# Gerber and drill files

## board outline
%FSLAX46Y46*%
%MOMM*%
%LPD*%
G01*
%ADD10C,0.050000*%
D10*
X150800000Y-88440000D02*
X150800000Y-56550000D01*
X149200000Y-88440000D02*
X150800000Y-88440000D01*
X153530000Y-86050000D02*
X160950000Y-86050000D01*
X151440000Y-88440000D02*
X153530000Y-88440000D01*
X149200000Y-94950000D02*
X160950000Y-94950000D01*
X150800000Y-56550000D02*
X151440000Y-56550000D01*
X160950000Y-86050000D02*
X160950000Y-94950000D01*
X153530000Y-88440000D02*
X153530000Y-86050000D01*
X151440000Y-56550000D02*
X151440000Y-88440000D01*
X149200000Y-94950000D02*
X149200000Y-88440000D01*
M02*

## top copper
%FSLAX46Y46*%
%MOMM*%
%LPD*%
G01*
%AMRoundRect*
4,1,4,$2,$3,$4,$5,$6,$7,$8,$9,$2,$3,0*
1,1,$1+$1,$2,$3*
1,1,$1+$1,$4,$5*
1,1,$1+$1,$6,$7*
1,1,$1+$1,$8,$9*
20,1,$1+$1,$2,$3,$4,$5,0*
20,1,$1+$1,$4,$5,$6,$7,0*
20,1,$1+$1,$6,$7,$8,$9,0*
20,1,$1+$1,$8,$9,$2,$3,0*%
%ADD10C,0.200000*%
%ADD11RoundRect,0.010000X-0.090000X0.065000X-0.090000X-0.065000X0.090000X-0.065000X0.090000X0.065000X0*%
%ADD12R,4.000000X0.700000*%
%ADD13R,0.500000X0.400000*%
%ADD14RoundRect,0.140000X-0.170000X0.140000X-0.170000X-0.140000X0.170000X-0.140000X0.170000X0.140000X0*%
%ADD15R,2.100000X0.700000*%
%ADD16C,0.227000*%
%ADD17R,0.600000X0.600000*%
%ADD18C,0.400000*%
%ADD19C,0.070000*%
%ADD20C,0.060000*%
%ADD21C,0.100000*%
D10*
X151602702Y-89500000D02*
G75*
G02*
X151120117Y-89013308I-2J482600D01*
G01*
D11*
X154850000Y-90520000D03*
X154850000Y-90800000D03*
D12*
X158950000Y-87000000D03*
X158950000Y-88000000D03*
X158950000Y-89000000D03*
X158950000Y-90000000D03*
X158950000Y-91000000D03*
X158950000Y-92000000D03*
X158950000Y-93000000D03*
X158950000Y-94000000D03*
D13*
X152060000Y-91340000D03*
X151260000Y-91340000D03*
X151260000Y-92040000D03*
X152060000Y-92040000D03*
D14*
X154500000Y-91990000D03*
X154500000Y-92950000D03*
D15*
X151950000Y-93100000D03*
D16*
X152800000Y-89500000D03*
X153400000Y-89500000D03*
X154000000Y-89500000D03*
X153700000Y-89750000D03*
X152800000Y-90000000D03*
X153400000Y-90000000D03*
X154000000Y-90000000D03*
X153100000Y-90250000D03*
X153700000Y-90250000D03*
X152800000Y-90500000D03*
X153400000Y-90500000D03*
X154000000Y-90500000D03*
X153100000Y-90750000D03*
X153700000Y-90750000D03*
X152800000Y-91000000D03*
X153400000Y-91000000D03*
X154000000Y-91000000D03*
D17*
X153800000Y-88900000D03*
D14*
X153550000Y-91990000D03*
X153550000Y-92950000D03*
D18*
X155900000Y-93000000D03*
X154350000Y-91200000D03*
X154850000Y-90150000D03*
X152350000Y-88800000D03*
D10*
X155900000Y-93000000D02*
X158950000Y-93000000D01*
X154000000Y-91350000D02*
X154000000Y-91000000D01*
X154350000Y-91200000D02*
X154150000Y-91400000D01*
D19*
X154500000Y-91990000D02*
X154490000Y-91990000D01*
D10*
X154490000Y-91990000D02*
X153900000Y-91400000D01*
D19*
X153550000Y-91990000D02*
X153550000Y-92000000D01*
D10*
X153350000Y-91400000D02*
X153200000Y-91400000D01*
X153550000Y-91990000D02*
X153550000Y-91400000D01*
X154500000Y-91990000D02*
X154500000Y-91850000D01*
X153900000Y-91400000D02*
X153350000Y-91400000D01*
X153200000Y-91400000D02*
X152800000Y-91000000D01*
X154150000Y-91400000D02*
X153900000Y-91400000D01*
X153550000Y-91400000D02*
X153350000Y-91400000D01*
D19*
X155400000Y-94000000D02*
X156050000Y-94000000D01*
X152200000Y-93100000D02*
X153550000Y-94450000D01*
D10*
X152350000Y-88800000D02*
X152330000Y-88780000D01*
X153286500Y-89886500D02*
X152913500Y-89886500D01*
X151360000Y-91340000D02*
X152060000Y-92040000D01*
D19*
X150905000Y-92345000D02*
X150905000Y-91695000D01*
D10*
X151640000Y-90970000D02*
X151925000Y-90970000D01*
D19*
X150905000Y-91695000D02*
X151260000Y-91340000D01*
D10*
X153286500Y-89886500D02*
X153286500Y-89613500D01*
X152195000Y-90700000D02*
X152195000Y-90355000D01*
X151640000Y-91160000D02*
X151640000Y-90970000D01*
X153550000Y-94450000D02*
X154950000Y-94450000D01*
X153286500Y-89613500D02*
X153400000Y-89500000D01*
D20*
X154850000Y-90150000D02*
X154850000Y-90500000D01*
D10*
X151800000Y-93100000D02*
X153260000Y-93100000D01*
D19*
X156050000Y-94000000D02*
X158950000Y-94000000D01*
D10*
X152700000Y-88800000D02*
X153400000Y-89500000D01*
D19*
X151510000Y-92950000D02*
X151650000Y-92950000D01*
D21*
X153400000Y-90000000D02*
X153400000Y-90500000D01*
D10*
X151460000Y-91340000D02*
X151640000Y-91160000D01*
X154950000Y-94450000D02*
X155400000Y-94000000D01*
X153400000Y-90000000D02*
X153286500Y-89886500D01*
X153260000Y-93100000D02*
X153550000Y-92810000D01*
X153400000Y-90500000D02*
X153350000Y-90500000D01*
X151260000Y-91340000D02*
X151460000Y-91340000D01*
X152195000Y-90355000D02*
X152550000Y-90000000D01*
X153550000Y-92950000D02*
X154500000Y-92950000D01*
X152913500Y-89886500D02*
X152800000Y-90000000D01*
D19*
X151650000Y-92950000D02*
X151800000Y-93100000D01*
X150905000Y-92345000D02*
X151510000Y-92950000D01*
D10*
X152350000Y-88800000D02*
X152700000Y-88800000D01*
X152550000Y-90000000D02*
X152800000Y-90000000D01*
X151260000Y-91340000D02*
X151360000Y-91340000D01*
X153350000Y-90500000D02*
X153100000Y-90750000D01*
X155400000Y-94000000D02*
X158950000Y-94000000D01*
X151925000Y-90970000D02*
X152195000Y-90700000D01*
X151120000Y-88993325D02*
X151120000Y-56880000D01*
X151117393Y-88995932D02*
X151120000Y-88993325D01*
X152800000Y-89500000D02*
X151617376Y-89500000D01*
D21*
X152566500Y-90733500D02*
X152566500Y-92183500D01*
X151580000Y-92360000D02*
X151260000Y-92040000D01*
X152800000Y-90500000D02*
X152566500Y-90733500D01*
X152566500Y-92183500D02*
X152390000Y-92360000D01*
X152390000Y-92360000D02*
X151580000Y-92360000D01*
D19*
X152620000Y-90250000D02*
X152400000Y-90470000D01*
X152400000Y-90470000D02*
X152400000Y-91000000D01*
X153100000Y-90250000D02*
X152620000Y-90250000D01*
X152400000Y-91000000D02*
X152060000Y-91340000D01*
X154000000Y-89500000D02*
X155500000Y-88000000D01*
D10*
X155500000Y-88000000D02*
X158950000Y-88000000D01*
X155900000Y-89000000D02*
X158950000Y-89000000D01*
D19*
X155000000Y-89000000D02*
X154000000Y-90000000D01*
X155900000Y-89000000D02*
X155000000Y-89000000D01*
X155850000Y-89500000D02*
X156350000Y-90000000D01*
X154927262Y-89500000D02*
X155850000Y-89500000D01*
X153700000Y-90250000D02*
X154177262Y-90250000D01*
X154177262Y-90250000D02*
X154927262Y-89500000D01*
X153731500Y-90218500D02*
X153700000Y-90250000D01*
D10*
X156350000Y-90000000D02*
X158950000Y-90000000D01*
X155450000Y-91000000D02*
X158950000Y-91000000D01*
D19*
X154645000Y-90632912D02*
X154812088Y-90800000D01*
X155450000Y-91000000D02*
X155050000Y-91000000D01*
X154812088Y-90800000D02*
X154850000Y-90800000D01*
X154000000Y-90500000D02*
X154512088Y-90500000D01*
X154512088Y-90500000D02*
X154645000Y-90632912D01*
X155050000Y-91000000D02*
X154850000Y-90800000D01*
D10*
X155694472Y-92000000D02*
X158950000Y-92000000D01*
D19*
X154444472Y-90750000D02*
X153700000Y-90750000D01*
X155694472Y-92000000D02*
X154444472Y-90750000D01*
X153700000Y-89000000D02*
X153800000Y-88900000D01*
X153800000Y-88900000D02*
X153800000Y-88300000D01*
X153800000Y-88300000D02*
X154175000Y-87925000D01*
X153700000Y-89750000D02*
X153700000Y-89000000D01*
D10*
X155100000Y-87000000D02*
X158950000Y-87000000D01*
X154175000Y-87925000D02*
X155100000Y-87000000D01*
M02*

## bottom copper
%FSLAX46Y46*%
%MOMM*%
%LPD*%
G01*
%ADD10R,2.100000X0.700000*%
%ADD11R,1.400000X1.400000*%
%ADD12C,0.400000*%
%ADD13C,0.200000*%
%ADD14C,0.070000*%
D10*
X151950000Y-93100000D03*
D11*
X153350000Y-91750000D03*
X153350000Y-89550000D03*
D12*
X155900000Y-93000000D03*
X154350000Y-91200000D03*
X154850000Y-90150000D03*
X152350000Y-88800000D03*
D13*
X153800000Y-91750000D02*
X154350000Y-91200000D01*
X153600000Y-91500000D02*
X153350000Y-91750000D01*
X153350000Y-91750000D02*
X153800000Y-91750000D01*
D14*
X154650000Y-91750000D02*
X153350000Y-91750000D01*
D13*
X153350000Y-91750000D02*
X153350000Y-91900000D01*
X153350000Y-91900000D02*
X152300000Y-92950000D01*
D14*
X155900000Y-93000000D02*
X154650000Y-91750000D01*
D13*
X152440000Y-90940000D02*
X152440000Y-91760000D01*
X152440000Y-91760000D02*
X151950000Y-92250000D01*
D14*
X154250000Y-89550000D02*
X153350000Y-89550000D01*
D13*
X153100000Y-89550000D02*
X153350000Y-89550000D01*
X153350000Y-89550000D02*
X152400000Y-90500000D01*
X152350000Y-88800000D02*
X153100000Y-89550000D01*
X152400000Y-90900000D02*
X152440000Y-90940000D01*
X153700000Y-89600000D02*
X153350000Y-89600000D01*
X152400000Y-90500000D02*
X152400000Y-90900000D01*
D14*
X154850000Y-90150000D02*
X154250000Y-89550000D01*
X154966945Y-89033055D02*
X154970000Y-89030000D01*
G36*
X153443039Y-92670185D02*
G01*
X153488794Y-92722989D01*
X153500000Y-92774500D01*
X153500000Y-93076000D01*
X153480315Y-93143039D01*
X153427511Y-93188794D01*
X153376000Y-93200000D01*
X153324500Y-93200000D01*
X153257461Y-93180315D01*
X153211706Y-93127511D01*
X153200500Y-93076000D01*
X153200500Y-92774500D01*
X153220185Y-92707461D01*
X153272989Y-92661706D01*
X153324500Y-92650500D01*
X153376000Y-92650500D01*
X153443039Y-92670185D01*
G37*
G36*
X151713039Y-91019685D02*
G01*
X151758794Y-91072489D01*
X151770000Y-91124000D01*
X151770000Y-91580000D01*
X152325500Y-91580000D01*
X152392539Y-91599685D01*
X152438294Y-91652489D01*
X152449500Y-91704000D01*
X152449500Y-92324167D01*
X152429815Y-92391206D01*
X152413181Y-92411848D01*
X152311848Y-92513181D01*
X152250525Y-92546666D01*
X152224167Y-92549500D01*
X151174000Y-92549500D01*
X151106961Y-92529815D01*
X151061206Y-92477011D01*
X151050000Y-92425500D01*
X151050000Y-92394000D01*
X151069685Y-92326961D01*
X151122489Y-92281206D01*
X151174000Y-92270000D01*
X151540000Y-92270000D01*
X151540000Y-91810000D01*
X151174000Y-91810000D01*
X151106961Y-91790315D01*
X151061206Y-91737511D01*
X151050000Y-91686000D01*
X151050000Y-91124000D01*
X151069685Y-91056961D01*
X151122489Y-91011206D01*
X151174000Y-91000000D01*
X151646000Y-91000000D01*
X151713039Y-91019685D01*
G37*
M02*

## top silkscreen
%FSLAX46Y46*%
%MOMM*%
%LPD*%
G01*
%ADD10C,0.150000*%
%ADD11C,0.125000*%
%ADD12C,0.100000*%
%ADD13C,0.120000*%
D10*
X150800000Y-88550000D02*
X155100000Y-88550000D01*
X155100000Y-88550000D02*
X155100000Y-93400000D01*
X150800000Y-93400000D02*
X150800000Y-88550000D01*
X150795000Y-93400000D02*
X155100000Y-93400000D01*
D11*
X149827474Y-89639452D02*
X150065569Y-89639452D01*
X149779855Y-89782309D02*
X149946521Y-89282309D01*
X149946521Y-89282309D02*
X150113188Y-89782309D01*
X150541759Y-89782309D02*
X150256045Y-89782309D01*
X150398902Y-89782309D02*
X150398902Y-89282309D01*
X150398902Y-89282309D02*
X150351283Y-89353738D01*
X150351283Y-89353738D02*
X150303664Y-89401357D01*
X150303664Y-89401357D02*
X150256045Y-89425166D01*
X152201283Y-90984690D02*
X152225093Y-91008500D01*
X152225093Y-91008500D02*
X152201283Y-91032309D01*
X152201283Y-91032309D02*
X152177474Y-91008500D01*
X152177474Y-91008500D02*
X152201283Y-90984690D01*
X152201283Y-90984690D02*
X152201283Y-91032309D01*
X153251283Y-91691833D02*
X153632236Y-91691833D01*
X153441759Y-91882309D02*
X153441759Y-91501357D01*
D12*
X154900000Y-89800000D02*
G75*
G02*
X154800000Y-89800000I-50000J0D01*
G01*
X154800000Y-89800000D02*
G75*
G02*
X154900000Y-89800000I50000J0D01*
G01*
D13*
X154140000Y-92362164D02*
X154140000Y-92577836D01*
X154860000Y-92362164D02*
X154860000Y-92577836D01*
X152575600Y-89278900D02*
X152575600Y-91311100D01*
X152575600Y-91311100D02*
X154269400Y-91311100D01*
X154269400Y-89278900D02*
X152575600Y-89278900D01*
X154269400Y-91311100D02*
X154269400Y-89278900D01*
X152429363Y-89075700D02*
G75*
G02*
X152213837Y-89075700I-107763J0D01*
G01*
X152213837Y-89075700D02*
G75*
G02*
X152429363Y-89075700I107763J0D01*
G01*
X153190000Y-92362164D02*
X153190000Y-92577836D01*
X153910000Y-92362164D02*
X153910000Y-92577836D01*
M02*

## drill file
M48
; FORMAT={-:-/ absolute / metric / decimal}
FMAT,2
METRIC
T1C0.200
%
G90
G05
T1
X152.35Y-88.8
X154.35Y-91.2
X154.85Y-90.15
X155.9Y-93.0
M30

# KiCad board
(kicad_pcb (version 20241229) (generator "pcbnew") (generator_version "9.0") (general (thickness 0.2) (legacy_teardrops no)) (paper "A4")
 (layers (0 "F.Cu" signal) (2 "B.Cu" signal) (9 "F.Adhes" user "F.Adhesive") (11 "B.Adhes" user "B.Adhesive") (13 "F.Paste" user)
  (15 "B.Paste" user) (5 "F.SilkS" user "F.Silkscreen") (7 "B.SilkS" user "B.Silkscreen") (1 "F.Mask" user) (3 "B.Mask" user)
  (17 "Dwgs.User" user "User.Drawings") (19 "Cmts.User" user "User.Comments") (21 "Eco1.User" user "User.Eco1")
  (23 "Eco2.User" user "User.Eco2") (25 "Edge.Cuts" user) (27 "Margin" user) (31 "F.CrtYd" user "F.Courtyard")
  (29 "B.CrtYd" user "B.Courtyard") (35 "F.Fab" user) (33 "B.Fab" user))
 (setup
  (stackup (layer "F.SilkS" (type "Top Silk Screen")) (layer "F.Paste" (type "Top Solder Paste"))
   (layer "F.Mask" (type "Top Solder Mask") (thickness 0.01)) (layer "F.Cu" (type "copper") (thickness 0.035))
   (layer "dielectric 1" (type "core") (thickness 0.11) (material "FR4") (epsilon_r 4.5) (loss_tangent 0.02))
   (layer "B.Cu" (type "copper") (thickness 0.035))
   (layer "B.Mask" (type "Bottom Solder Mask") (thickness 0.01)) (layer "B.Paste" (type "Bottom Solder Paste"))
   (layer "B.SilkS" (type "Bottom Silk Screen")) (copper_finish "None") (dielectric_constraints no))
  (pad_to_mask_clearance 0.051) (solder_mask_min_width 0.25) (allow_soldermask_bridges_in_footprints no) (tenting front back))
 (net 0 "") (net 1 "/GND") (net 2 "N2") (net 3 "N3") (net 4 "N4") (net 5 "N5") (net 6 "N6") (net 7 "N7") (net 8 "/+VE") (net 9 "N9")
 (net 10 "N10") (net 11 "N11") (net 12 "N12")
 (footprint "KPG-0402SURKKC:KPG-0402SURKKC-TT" (layer "F.Cu") (at 154.85 90.66 -90)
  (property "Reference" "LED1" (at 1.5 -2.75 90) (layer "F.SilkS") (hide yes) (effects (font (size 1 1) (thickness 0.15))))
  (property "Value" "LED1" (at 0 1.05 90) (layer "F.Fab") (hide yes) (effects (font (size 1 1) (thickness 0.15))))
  (fp_circle (center -0.86 0) (end -0.81 0) (stroke (width 0.1) (type solid)) (fill no) (layer "F.SilkS"))
  (pad "" smd roundrect (at -0.14 0 270) (size 0.15 0.2) (layers "F.Mask") (roundrect_rratio 0.06666666667))
  (pad "" smd roundrect (at -0.1225 0 270) (size 0.1 0.17) (layers "F.Paste") (roundrect_rratio 0.25))
  (pad "" smd roundrect (at 0.1225 0 270) (size 0.1 0.17) (layers "F.Paste") (roundrect_rratio 0.25))
  (pad "" smd roundrect (at 0.14 0 270) (size 0.15 0.2) (layers "F.Mask") (roundrect_rratio 0.06666666667))
  (pad "1" smd roundrect (at -0.14 0 270) (size 0.15 0.2) (layers "F.Cu" "F.Mask") (roundrect_rratio 0.06666666667) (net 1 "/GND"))
  (pad "2" smd roundrect (at 0.14 0 270) (size 0.15 0.2) (layers "F.Cu" "F.Mask") (roundrect_rratio 0.06666666667) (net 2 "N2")))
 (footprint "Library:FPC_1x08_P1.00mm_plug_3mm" (layer "F.Cu") (at 156.95 90.5)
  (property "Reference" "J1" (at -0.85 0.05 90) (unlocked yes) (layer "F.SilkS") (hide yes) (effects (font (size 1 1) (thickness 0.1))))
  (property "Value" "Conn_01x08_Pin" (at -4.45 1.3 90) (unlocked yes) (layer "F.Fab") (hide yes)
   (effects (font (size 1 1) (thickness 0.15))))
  (pad "1" connect rect (at 2 -3.5) (size 4 0.7) (layers "F.Cu" "F.Mask") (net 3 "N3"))
  (pad "2" connect rect (at 2 -2.5) (size 4 0.7) (layers "F.Cu" "F.Mask") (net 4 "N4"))
  (pad "3" connect rect (at 2 -1.5) (size 4 0.7) (layers "F.Cu" "F.Mask") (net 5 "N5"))
  (pad "4" connect rect (at 2 -0.5) (size 4 0.7) (layers "F.Cu" "F.Mask") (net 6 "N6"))
  (pad "5" connect rect (at 2 0.5) (size 4 0.7) (layers "F.Cu" "F.Mask") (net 2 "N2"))
  (pad "6" connect rect (at 2 1.5) (size 4 0.7) (layers "F.Cu" "F.Mask") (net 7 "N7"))
  (pad "7" connect rect (at 2 2.5) (size 4 0.7) (layers "F.Cu" "F.Mask") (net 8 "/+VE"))
  (pad "8" connect rect (at 2 3.5) (size 4 0.7) (layers "F.Cu" "F.Mask") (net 1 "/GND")))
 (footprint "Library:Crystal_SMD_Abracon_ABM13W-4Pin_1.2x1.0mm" (layer "F.Cu") (at 151.66 91.69 180)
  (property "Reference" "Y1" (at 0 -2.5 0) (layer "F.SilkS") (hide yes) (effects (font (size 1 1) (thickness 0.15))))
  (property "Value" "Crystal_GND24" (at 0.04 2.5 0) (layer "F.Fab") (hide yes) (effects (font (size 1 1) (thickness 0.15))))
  (pad "1" smd rect (at -0.4 0.35 180) (size 0.5 0.4) (layers "F.Cu" "F.Mask" "F.Paste") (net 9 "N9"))
  (pad "2" smd rect (at 0.4 0.35 180) (size 0.5 0.4) (layers "F.Cu" "F.Mask" "F.Paste") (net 1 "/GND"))
  (pad "3" smd rect (at 0.4 -0.35 180) (size 0.5 0.4) (layers "F.Cu" "F.Mask" "F.Paste") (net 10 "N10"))
  (pad "4" smd rect (at -0.4 -0.35 180) (size 0.5 0.4) (layers "F.Cu" "F.Mask" "F.Paste") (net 1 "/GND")))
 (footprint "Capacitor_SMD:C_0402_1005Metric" (layer "F.Cu") (at 154.5 92.47 -90)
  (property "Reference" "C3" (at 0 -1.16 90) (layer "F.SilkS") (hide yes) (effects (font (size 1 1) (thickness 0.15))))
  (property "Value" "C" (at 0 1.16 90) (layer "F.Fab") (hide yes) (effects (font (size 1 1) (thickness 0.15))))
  (fp_line (start -0.107836 0.36) (end 0.107836 0.36) (stroke (width 0.12) (type solid)) (layer "F.SilkS"))
  (fp_line (start -0.107836 -0.36) (end 0.107836 -0.36) (stroke (width 0.12) (type solid)) (layer "F.SilkS"))
  (pad "1" smd roundrect (at -0.48 0 270) (size 0.56 0.62) (layers "F.Cu" "F.Mask" "F.Paste") (roundrect_rratio 0.25) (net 8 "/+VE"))
  (pad "2" smd roundrect (at 0.48 0 270) (size 0.56 0.62) (layers "F.Cu" "F.Mask" "F.Paste") (roundrect_rratio 0.25) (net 1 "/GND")))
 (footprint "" (layer "F.Cu") (at 153.4 91.95)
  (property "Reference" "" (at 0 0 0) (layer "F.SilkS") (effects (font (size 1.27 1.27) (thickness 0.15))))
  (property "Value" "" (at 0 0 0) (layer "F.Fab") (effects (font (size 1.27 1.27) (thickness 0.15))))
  (pad "1" smd rect (at -1.45 1.15) (size 2.1 0.7) (layers "F.Cu" "F.Mask") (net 1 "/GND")))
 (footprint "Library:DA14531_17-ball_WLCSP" (layer "F.Cu") (at 153.422 90.295)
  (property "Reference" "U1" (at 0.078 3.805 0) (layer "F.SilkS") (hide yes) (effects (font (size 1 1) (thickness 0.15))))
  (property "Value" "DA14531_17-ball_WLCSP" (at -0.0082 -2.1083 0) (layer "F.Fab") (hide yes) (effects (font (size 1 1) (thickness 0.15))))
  (fp_line (start -0.8464 -1.0161) (end -0.8464 1.0161) (stroke (width 0.12) (type solid)) (layer "F.SilkS"))
  (fp_line (start -0.8464 1.0161) (end 0.8474 1.0161) (stroke (width 0.12) (type solid)) (layer "F.SilkS"))
  (fp_line (start 0.8474 -1.0161) (end -0.8464 -1.0161) (stroke (width 0.12) (type solid)) (layer "F.SilkS"))
  (fp_line (start 0.8474 1.0161) (end 0.8474 -1.0161) (stroke (width 0.12) (type solid)) (layer "F.SilkS"))
  (fp_circle (center -1.1004 -1.2193) (end -1.0242 -1.1431) (stroke (width 0.12) (type solid)) (fill no) (layer "F.SilkS"))
  (pad "A1" smd circle (at -0.622 -0.795) (size 0.227 0.227) (layers "F.Cu" "F.Mask" "F.Paste") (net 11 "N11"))
  (pad "A3" smd circle (at -0.022 -0.795) (size 0.227 0.227) (layers "F.Cu" "F.Mask" "F.Paste") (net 1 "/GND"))
  (pad "A5" smd circle (at 0.578 -0.795) (size 0.227 0.227) (layers "F.Cu" "F.Mask" "F.Paste") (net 4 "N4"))
  (pad "B4" smd circle (at 0.278 -0.545) (size 0.227 0.227) (layers "F.Cu" "F.Mask" "F.Paste") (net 3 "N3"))
  (pad "C1" smd circle (at -0.622 -0.295) (size 0.227 0.227) (layers "F.Cu" "F.Mask" "F.Paste") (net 1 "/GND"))
  (pad "C3" smd circle (at -0.022 -0.295) (size 0.227 0.227) (layers "F.Cu" "F.Mask" "F.Paste") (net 1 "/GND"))
  (pad "C5" smd circle (at 0.578 -0.295) (size 0.227 0.227) (layers "F.Cu" "F.Mask" "F.Paste") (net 5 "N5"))
  (pad "D2" smd circle (at -0.322 -0.045) (size 0.227 0.227) (layers "F.Cu" "F.Mask" "F.Paste") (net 9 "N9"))
  (pad "D4" smd circle (at 0.278 -0.045) (size 0.227 0.227) (layers "F.Cu" "F.Mask" "F.Paste") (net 6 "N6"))
  (pad "E1" smd circle (at -0.622 0.205) (size 0.227 0.227) (layers "F.Cu" "F.Mask" "F.Paste") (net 10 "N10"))
  (pad "E3" smd circle (at -0.022 0.205) (size 0.227 0.227) (layers "F.Cu" "F.Mask" "F.Paste") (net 1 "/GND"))
  (pad "E5" smd circle (at 0.578 0.205) (size 0.227 0.227) (layers "F.Cu" "F.Mask" "F.Paste") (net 2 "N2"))
  (pad "F2" smd circle (at -0.322 0.455) (size 0.227 0.227) (layers "F.Cu" "F.Mask" "F.Paste") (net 1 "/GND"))
  (pad "F4" smd circle (at 0.278 0.455) (size 0.227 0.227) (layers "F.Cu" "F.Mask" "F.Paste") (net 7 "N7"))
  (pad "G1" smd circle (at -0.622 0.705) (size 0.227 0.227) (layers "F.Cu" "F.Mask" "F.Paste") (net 8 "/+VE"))
  (pad "G3" smd circle (at -0.022 0.705) (size 0.227 0.227) (layers "F.Cu" "F.Mask" "F.Paste") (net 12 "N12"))
  (pad "G5" smd circle (at 0.578 0.705) (size 0.227 0.227) (layers "F.Cu" "F.Mask" "F.Paste") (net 8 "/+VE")))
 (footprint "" (layer "F.Cu") (at 156 87.8)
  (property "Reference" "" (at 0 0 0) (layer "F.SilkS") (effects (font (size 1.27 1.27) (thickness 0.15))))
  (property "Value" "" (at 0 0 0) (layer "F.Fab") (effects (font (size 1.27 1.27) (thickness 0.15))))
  (pad "1" smd rect (at -2.2 1.1) (size 0.6 0.6) (layers "F.Cu" "F.Mask") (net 3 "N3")))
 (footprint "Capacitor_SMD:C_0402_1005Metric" (layer "F.Cu") (at 153.55 92.47 -90)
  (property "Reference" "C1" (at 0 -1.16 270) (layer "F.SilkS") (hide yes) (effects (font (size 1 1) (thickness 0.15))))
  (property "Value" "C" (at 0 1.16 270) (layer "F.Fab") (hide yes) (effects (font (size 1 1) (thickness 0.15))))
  (fp_line (start -0.107836 0.36) (end 0.107836 0.36) (stroke (width 0.12) (type solid)) (layer "F.SilkS"))
  (fp_line (start -0.107836 -0.36) (end 0.107836 -0.36) (stroke (width 0.12) (type solid)) (layer "F.SilkS"))
  (pad "1" smd roundrect (at -0.48 0 270) (size 0.56 0.62) (layers "F.Cu" "F.Mask" "F.Paste") (roundrect_rratio 0.25) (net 8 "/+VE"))
  (pad "2" smd roundrect (at 0.48 0 270) (size 0.56 0.62) (layers "F.Cu" "F.Mask" "F.Paste") (roundrect_rratio 0.25) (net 1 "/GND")))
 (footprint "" (layer "B.Cu") (at 150.5 91.95 180)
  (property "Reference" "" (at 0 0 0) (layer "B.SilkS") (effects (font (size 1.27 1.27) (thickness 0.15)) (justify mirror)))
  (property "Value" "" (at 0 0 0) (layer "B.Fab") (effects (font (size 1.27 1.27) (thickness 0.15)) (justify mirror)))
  (pad "1" smd rect (at -1.45 -1.15 180) (size 2.1 0.7) (layers "B.Cu" "B.Mask") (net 8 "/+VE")))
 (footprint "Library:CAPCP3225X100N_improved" (layer "B.Cu") (at 153.35 90.65 90)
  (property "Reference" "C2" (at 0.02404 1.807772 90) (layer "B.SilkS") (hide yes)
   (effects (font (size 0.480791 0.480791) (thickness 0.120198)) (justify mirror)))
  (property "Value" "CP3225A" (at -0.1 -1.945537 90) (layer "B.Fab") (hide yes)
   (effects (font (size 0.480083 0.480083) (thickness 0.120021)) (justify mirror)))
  (pad "1" smd rect (at -1.1 0 270) (size 1.4 1.4) (layers "B.Cu" "B.Mask" "B.Paste") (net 8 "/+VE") (solder_mask_margin 0.102))
  (pad "2" smd rect (at 1.1 0 270) (size 1.4 1.4) (layers "B.Cu" "B.Mask" "B.Paste") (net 1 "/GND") (solder_mask_margin 0.102)))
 (gr_arc (start 151.602702 89.5) (mid 151.26 89.357201) (end 151.120095 89.013308) (stroke (width 0.2) (type default)) (layer "F.Cu")
  (net 11))
 (gr_line (start 150.8 88.55) (end 155.1 88.55) (stroke (width 0.15) (type default)) (layer "F.SilkS"))
 (gr_line (start 155.1 88.55) (end 155.1 93.4) (stroke (width 0.15) (type default)) (layer "F.SilkS"))
 (gr_line (start 150.8 93.4) (end 150.8 88.55) (stroke (width 0.15) (type default)) (layer "F.SilkS"))
 (gr_line (start 150.795 93.4) (end 155.1 93.4) (stroke (width 0.15) (type default)) (layer "F.SilkS"))
 (gr_line (start 150.8 88.44) (end 150.8 56.55) (stroke (width 0.05) (type default)) (layer "Edge.Cuts"))
 (gr_line (start 149.2 88.44) (end 150.8 88.44) (stroke (width 0.05) (type default)) (layer "Edge.Cuts"))
 (gr_line (start 153.53 86.05) (end 160.95 86.05) (stroke (width 0.05) (type default)) (layer "Edge.Cuts"))
 (gr_line (start 151.44 88.44) (end 153.53 88.44) (stroke (width 0.05) (type default)) (layer "Edge.Cuts"))
 (gr_line (start 149.2 94.95) (end 160.95 94.95) (stroke (width 0.05) (type default)) (layer "Edge.Cuts"))
 (gr_line (start 150.8 56.55) (end 151.44 56.55) (stroke (width 0.05) (type default)) (layer "Edge.Cuts"))
 (gr_line (start 160.95 86.05) (end 160.95 94.95) (stroke (width 0.05) (type default)) (layer "Edge.Cuts"))
 (gr_line (start 153.53 88.44) (end 153.53 86.05) (stroke (width 0.05) (type default)) (layer "Edge.Cuts"))
 (gr_line (start 151.44 56.55) (end 151.44 88.44) (stroke (width 0.05) (type default)) (layer "Edge.Cuts"))
 (gr_line (start 149.2 94.95) (end 149.2 88.44) (stroke (width 0.05) (type default)) (layer "Edge.Cuts"))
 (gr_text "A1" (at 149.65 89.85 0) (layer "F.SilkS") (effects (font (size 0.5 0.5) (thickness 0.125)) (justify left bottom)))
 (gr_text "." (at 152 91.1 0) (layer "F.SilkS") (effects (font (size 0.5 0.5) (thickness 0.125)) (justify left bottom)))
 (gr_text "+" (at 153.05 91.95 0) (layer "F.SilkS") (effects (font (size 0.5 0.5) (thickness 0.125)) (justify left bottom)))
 (segment (start 155.9 93) (end 158.95 93) (width 0.2) (layer "F.Cu") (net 8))
 (segment (start 154 91.35) (end 154 91) (width 0.2) (layer "F.Cu") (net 8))
 (segment (start 154.35 91.2) (end 154.15 91.4) (width 0.2) (layer "F.Cu") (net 8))
 (segment (start 154.5 91.99) (end 154.49 91.99) (width 0.07) (layer "F.Cu") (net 8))
 (segment (start 154.49 91.99) (end 153.9 91.4) (width 0.2) (layer "F.Cu") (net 8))
 (segment (start 153.55 91.99) (end 153.55 92) (width 0.07) (layer "F.Cu") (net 8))
 (segment (start 153.35 91.4) (end 153.2 91.4) (width 0.2) (layer "F.Cu") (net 8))
 (segment (start 153.55 91.99) (end 153.55 91.4) (width 0.2) (layer "F.Cu") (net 8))
 (segment (start 154.5 91.99) (end 154.5 91.85) (width 0.2) (layer "F.Cu") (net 8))
 (segment (start 153.9 91.4) (end 153.35 91.4) (width 0.2) (layer "F.Cu") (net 8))
 (segment (start 153.2 91.4) (end 152.8 91) (width 0.2) (layer "F.Cu") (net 8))
 (segment (start 154.15 91.4) (end 153.9 91.4) (width 0.2) (layer "F.Cu") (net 8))
 (segment (start 153.55 91.4) (end 153.35 91.4) (width 0.2) (layer "F.Cu") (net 8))
 (via (at 155.9 93) (size 0.4) (drill 0.2) (layers "F.Cu" "B.Cu") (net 8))
 (via (at 154.35 91.2) (size 0.4) (drill 0.2) (layers "F.Cu" "B.Cu") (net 8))
 (segment (start 153.8 91.75) (end 154.35 91.2) (width 0.2) (layer "B.Cu") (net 8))
 (segment (start 153.6 91.5) (end 153.35 91.75) (width 0.2) (layer "B.Cu") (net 8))
 (segment (start 153.35 91.75) (end 153.8 91.75) (width 0.2) (layer "B.Cu") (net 8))
 (segment (start 154.65 91.75) (end 153.35 91.75) (width 0.07) (layer "B.Cu") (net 8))
 (segment (start 153.35 91.75) (end 153.35 91.9) (width 0.2) (layer "B.Cu") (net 8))
 (segment (start 153.35 91.9) (end 152.3 92.95) (width 0.2) (layer "B.Cu") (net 8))
 (segment (start 155.9 93) (end 154.65 91.75) (width 0.07) (layer "B.Cu") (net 8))
 (segment (start 155.4 94) (end 156.05 94) (width 0.07) (layer "F.Cu") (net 1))
 (segment (start 152.2 93.1) (end 153.55 94.45) (width 0.07) (layer "F.Cu") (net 1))
 (segment (start 152.35 88.8) (end 152.33 88.78) (width 0.2) (layer "F.Cu") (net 1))
 (segment (start 153.2865 89.8865) (end 152.9135 89.8865) (width 0.2) (layer "F.Cu") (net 1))
 (segment (start 151.36 91.34) (end 152.06 92.04) (width 0.2) (layer "F.Cu") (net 1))
 (segment (start 150.905 92.345) (end 150.905 91.695) (width 0.07) (layer "F.Cu") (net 1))
 (segment (start 151.64 90.97) (end 151.925 90.97) (width 0.2) (layer "F.Cu") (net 1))
 (segment (start 150.905 91.695) (end 151.26 91.34) (width 0.07) (layer "F.Cu") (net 1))
 (segment (start 153.2865 89.8865) (end 153.2865 89.6135) (width 0.2) (layer "F.Cu") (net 1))
 (segment (start 152.195 90.7) (end 152.195 90.355) (width 0.2) (layer "F.Cu") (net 1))
 (segment (start 151.64 91.16) (end 151.64 90.97) (width 0.2) (layer "F.Cu") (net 1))
 (segment (start 153.55 94.45) (end 154.95 94.45) (width 0.2) (layer "F.Cu") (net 1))
 (segment (start 153.2865 89.6135) (end 153.4 89.5) (width 0.2) (layer "F.Cu") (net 1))
 (segment (start 154.85 90.15) (end 154.85 90.5) (width 0.06) (layer "F.Cu") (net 1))
 (segment (start 151.8 93.1) (end 153.26 93.1) (width 0.2) (layer "F.Cu") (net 1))
 (segment (start 156.05 94) (end 158.95 94) (width 0.07) (layer "F.Cu") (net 1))
 (segment (start 152.7 88.8) (end 153.4 89.5) (width 0.2) (layer "F.Cu") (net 1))
 (segment (start 151.51 92.95) (end 151.65 92.95) (width 0.07) (layer "F.Cu") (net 1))
 (segment (start 153.4 90) (end 153.4 90.5) (width 0.1) (layer "F.Cu") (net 1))
 (segment (start 151.46 91.34) (end 151.64 91.16) (width 0.2) (layer "F.Cu") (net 1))
 (segment (start 154.95 94.45) (end 155.4 94) (width 0.2) (layer "F.Cu") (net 1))
 (segment (start 153.4 90) (end 153.2865 89.8865) (width 0.2) (layer "F.Cu") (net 1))
 (segment (start 153.26 93.1) (end 153.55 92.81) (width 0.2) (layer "F.Cu") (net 1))
 (segment (start 153.4 90.5) (end 153.35 90.5) (width 0.2) (layer "F.Cu") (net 1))
 (segment (start 151.26 91.34) (end 151.46 91.34) (width 0.2) (layer "F.Cu") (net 1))
 (segment (start 152.195 90.355) (end 152.55 90) (width 0.2) (layer "F.Cu") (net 1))
 (segment (start 153.55 92.95) (end 154.5 92.95) (width 0.2) (layer "F.Cu") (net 1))
 (segment (start 152.9135 89.8865) (end 152.8 90) (width 0.2) (layer "F.Cu") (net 1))
 (segment (start 151.65 92.95) (end 151.8 93.1) (width 0.07) (layer "F.Cu") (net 1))
 (segment (start 150.905 92.345) (end 151.51 92.95) (width 0.07) (layer "F.Cu") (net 1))
 (segment (start 152.35 88.8) (end 152.7 88.8) (width 0.2) (layer "F.Cu") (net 1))
 (segment (start 152.55 90) (end 152.8 90) (width 0.2) (layer "F.Cu") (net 1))
 (segment (start 151.26 91.34) (end 151.36 91.34) (width 0.2) (layer "F.Cu") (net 1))
 (segment (start 153.35 90.5) (end 153.1 90.75) (width 0.2) (layer "F.Cu") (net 1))
 (segment (start 155.4 94) (end 158.95 94) (width 0.2) (layer "F.Cu") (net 1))
 (segment (start 151.925 90.97) (end 152.195 90.7) (width 0.2) (layer "F.Cu") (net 1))
 (via (at 154.85 90.15) (size 0.4) (drill 0.2) (layers "F.Cu" "B.Cu") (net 1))
 (via (at 152.35 88.8) (size 0.4) (drill 0.2) (layers "F.Cu" "B.Cu") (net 1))
 (segment (start 152.44 90.94) (end 152.44 91.76) (width 0.2) (layer "B.Cu") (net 1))
 (segment (start 152.44 91.76) (end 151.95 92.25) (width 0.2) (layer "B.Cu") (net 1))
 (segment (start 154.25 89.55) (end 153.35 89.55) (width 0.07) (layer "B.Cu") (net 1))
 (segment (start 153.1 89.55) (end 153.35 89.55) (width 0.2) (layer "B.Cu") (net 1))
 (segment (start 153.35 89.55) (end 152.4 90.5) (width 0.2) (layer "B.Cu") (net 1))
 (segment (start 152.35 88.8) (end 153.1 89.55) (width 0.2) (layer "B.Cu") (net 1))
 (segment (start 152.4 90.9) (end 152.44 90.94) (width 0.2) (layer "B.Cu") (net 1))
 (segment (start 153.7 89.6) (end 153.35 89.6) (width 0.2) (layer "B.Cu") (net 1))
 (segment (start 152.4 90.5) (end 152.4 90.9) (width 0.2) (layer "B.Cu") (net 1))
 (segment (start 154.85 90.15) (end 154.25 89.55) (width 0.07) (layer "B.Cu") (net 1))
 (segment (start 151.12 88.993325) (end 151.12 56.88) (width 0.2) (layer "F.Cu") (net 11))
 (segment (start 151.117393 88.995932) (end 151.12 88.993325) (width 0.2) (layer "F.Cu") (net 11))
 (segment (start 152.8 89.5) (end 151.617376 89.5) (width 0.2) (layer "F.Cu") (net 11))
 (segment (start 152.5665 90.7335) (end 152.5665 92.1835) (width 0.1) (layer "F.Cu") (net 10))
 (segment (start 151.58 92.36) (end 151.26 92.04) (width 0.1) (layer "F.Cu") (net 10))
 (segment (start 152.8 90.5) (end 152.5665 90.7335) (width 0.1) (layer "F.Cu") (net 10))
 (segment (start 152.5665 92.1835) (end 152.39 92.36) (width 0.1) (layer "F.Cu") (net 10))
 (segment (start 152.39 92.36) (end 151.58 92.36) (width 0.1) (layer "F.Cu") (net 10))
 (segment (start 152.62 90.25) (end 152.4 90.47) (width 0.07) (layer "F.Cu") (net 9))
 (segment (start 152.4 90.47) (end 152.4 91) (width 0.07) (layer "F.Cu") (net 9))
 (segment (start 153.1 90.25) (end 152.62 90.25) (width 0.07) (layer "F.Cu") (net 9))
 (segment (start 152.4 91) (end 152.06 91.34) (width 0.07) (layer "F.Cu") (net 9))
 (segment (start 154 89.5) (end 155.5 88) (width 0.07) (layer "F.Cu") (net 4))
 (segment (start 155.5 88) (end 158.95 88) (width 0.2) (layer "F.Cu") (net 4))
 (segment (start 155.9 89) (end 158.95 89) (width 0.2) (layer "F.Cu") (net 5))
 (segment (start 155 89) (end 154 90) (width 0.07) (layer "F.Cu") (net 5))
 (segment (start 155.9 89) (end 155 89) (width 0.07) (layer "F.Cu") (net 5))
 (segment (start 154.966945 89.033055) (end 154.97 89.03) (width 0.07) (layer "B.Cu") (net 5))
 (segment (start 155.85 89.5) (end 156.35 90) (width 0.07) (layer "F.Cu") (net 6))
 (segment (start 154.927262 89.5) (end 155.85 89.5) (width 0.07) (layer "F.Cu") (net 6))
 (segment (start 153.7 90.25) (end 154.177262 90.25) (width 0.07) (layer "F.Cu") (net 6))
 (segment (start 154.177262 90.25) (end 154.927262 89.5) (width 0.07) (layer "F.Cu") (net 6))
 (segment (start 153.7315 90.2185) (end 153.7 90.25) (width 0.07) (layer "F.Cu") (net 6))
 (segment (start 156.35 90) (end 158.95 90) (width 0.2) (layer "F.Cu") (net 6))
 (segment (start 155.45 91) (end 158.95 91) (width 0.2) (layer "F.Cu") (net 2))
 (segment (start 154.645 90.632912) (end 154.812088 90.8) (width 0.07) (layer "F.Cu") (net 2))
 (segment (start 155.45 91) (end 155.05 91) (width 0.07) (layer "F.Cu") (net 2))
 (segment (start 154.812088 90.8) (end 154.85 90.8) (width 0.07) (layer "F.Cu") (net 2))
 (segment (start 154 90.5) (end 154.512088 90.5) (width 0.07) (layer "F.Cu") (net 2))
 (segment (start 154.512088 90.5) (end 154.645 90.632912) (width 0.07) (layer "F.Cu") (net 2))
 (segment (start 155.05 91) (end 154.85 90.8) (width 0.07) (layer "F.Cu") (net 2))
 (segment (start 155.694472 92) (end 158.95 92) (width 0.2) (layer "F.Cu") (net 7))
 (segment (start 154.444472 90.75) (end 153.7 90.75) (width 0.07) (layer "F.Cu") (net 7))
 (segment (start 155.694472 92) (end 154.444472 90.75) (width 0.07) (layer "F.Cu") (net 7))
 (segment (start 153.7 89) (end 153.8 88.9) (width 0.07) (layer "F.Cu") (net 3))
 (segment (start 153.8 88.9) (end 153.8 88.3) (width 0.07) (layer "F.Cu") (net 3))
 (segment (start 153.8 88.3) (end 154.175 87.925) (width 0.07) (layer "F.Cu") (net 3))
 (segment (start 153.7 89.75) (end 153.7 89) (width 0.07) (layer "F.Cu") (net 3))
 (segment (start 155.1 87) (end 158.95 87) (width 0.2) (layer "F.Cu") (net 3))
 (segment (start 154.175 87.925) (end 155.1 87) (width 0.2) (layer "F.Cu") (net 3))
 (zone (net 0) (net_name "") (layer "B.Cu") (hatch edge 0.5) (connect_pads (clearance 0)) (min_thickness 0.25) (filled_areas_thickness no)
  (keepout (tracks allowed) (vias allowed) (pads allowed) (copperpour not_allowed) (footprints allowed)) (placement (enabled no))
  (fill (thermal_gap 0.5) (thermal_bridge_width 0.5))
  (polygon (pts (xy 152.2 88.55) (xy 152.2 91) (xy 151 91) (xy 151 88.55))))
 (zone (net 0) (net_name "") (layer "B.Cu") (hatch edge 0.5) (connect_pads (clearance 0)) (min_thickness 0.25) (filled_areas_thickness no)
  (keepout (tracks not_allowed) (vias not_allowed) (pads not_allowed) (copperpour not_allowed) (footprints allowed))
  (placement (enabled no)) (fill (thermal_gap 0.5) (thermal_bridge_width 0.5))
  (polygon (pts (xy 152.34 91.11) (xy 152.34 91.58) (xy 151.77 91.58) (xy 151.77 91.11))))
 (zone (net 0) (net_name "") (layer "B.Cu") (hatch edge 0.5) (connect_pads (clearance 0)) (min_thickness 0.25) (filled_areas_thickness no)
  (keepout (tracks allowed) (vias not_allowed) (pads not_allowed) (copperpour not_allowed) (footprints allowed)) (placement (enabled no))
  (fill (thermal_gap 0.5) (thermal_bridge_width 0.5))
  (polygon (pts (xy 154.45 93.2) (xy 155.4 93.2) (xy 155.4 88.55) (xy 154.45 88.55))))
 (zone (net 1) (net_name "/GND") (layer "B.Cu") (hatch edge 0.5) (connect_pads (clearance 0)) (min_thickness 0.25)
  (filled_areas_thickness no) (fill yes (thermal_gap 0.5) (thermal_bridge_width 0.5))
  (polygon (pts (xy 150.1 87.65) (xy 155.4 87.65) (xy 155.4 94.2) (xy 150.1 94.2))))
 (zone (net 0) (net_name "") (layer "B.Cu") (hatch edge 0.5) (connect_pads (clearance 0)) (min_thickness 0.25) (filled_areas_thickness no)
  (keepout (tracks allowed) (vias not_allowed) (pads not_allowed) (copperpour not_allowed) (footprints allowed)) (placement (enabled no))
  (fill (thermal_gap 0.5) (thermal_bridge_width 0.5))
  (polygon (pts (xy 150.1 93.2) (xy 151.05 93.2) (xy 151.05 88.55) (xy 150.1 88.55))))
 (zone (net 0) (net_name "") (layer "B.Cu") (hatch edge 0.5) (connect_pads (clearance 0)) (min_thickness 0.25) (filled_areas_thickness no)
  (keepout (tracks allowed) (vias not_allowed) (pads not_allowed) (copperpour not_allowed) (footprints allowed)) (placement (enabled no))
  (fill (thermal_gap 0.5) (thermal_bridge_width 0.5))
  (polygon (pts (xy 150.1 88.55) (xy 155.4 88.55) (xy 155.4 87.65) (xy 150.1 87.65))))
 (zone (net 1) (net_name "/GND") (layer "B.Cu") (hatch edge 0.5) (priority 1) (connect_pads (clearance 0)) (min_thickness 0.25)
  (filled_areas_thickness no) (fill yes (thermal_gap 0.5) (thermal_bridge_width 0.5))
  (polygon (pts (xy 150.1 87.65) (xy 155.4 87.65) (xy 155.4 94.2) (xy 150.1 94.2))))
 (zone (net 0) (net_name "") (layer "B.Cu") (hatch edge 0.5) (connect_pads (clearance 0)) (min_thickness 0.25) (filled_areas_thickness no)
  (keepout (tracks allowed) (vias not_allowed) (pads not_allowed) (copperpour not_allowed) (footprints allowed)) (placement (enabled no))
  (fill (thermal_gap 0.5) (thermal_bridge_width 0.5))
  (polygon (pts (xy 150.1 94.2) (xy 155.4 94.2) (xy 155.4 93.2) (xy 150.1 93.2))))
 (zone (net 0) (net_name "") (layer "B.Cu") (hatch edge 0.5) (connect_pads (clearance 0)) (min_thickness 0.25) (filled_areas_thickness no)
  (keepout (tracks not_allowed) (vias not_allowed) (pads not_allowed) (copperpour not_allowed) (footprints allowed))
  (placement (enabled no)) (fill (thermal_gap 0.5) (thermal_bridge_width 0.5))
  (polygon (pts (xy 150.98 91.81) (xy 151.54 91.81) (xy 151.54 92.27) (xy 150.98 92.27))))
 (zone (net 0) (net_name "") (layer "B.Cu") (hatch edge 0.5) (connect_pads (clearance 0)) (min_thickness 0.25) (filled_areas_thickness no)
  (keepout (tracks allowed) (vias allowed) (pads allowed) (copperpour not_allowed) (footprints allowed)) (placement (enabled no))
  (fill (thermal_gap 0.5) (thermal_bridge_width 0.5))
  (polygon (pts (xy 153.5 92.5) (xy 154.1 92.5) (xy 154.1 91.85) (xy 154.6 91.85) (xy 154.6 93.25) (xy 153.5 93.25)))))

